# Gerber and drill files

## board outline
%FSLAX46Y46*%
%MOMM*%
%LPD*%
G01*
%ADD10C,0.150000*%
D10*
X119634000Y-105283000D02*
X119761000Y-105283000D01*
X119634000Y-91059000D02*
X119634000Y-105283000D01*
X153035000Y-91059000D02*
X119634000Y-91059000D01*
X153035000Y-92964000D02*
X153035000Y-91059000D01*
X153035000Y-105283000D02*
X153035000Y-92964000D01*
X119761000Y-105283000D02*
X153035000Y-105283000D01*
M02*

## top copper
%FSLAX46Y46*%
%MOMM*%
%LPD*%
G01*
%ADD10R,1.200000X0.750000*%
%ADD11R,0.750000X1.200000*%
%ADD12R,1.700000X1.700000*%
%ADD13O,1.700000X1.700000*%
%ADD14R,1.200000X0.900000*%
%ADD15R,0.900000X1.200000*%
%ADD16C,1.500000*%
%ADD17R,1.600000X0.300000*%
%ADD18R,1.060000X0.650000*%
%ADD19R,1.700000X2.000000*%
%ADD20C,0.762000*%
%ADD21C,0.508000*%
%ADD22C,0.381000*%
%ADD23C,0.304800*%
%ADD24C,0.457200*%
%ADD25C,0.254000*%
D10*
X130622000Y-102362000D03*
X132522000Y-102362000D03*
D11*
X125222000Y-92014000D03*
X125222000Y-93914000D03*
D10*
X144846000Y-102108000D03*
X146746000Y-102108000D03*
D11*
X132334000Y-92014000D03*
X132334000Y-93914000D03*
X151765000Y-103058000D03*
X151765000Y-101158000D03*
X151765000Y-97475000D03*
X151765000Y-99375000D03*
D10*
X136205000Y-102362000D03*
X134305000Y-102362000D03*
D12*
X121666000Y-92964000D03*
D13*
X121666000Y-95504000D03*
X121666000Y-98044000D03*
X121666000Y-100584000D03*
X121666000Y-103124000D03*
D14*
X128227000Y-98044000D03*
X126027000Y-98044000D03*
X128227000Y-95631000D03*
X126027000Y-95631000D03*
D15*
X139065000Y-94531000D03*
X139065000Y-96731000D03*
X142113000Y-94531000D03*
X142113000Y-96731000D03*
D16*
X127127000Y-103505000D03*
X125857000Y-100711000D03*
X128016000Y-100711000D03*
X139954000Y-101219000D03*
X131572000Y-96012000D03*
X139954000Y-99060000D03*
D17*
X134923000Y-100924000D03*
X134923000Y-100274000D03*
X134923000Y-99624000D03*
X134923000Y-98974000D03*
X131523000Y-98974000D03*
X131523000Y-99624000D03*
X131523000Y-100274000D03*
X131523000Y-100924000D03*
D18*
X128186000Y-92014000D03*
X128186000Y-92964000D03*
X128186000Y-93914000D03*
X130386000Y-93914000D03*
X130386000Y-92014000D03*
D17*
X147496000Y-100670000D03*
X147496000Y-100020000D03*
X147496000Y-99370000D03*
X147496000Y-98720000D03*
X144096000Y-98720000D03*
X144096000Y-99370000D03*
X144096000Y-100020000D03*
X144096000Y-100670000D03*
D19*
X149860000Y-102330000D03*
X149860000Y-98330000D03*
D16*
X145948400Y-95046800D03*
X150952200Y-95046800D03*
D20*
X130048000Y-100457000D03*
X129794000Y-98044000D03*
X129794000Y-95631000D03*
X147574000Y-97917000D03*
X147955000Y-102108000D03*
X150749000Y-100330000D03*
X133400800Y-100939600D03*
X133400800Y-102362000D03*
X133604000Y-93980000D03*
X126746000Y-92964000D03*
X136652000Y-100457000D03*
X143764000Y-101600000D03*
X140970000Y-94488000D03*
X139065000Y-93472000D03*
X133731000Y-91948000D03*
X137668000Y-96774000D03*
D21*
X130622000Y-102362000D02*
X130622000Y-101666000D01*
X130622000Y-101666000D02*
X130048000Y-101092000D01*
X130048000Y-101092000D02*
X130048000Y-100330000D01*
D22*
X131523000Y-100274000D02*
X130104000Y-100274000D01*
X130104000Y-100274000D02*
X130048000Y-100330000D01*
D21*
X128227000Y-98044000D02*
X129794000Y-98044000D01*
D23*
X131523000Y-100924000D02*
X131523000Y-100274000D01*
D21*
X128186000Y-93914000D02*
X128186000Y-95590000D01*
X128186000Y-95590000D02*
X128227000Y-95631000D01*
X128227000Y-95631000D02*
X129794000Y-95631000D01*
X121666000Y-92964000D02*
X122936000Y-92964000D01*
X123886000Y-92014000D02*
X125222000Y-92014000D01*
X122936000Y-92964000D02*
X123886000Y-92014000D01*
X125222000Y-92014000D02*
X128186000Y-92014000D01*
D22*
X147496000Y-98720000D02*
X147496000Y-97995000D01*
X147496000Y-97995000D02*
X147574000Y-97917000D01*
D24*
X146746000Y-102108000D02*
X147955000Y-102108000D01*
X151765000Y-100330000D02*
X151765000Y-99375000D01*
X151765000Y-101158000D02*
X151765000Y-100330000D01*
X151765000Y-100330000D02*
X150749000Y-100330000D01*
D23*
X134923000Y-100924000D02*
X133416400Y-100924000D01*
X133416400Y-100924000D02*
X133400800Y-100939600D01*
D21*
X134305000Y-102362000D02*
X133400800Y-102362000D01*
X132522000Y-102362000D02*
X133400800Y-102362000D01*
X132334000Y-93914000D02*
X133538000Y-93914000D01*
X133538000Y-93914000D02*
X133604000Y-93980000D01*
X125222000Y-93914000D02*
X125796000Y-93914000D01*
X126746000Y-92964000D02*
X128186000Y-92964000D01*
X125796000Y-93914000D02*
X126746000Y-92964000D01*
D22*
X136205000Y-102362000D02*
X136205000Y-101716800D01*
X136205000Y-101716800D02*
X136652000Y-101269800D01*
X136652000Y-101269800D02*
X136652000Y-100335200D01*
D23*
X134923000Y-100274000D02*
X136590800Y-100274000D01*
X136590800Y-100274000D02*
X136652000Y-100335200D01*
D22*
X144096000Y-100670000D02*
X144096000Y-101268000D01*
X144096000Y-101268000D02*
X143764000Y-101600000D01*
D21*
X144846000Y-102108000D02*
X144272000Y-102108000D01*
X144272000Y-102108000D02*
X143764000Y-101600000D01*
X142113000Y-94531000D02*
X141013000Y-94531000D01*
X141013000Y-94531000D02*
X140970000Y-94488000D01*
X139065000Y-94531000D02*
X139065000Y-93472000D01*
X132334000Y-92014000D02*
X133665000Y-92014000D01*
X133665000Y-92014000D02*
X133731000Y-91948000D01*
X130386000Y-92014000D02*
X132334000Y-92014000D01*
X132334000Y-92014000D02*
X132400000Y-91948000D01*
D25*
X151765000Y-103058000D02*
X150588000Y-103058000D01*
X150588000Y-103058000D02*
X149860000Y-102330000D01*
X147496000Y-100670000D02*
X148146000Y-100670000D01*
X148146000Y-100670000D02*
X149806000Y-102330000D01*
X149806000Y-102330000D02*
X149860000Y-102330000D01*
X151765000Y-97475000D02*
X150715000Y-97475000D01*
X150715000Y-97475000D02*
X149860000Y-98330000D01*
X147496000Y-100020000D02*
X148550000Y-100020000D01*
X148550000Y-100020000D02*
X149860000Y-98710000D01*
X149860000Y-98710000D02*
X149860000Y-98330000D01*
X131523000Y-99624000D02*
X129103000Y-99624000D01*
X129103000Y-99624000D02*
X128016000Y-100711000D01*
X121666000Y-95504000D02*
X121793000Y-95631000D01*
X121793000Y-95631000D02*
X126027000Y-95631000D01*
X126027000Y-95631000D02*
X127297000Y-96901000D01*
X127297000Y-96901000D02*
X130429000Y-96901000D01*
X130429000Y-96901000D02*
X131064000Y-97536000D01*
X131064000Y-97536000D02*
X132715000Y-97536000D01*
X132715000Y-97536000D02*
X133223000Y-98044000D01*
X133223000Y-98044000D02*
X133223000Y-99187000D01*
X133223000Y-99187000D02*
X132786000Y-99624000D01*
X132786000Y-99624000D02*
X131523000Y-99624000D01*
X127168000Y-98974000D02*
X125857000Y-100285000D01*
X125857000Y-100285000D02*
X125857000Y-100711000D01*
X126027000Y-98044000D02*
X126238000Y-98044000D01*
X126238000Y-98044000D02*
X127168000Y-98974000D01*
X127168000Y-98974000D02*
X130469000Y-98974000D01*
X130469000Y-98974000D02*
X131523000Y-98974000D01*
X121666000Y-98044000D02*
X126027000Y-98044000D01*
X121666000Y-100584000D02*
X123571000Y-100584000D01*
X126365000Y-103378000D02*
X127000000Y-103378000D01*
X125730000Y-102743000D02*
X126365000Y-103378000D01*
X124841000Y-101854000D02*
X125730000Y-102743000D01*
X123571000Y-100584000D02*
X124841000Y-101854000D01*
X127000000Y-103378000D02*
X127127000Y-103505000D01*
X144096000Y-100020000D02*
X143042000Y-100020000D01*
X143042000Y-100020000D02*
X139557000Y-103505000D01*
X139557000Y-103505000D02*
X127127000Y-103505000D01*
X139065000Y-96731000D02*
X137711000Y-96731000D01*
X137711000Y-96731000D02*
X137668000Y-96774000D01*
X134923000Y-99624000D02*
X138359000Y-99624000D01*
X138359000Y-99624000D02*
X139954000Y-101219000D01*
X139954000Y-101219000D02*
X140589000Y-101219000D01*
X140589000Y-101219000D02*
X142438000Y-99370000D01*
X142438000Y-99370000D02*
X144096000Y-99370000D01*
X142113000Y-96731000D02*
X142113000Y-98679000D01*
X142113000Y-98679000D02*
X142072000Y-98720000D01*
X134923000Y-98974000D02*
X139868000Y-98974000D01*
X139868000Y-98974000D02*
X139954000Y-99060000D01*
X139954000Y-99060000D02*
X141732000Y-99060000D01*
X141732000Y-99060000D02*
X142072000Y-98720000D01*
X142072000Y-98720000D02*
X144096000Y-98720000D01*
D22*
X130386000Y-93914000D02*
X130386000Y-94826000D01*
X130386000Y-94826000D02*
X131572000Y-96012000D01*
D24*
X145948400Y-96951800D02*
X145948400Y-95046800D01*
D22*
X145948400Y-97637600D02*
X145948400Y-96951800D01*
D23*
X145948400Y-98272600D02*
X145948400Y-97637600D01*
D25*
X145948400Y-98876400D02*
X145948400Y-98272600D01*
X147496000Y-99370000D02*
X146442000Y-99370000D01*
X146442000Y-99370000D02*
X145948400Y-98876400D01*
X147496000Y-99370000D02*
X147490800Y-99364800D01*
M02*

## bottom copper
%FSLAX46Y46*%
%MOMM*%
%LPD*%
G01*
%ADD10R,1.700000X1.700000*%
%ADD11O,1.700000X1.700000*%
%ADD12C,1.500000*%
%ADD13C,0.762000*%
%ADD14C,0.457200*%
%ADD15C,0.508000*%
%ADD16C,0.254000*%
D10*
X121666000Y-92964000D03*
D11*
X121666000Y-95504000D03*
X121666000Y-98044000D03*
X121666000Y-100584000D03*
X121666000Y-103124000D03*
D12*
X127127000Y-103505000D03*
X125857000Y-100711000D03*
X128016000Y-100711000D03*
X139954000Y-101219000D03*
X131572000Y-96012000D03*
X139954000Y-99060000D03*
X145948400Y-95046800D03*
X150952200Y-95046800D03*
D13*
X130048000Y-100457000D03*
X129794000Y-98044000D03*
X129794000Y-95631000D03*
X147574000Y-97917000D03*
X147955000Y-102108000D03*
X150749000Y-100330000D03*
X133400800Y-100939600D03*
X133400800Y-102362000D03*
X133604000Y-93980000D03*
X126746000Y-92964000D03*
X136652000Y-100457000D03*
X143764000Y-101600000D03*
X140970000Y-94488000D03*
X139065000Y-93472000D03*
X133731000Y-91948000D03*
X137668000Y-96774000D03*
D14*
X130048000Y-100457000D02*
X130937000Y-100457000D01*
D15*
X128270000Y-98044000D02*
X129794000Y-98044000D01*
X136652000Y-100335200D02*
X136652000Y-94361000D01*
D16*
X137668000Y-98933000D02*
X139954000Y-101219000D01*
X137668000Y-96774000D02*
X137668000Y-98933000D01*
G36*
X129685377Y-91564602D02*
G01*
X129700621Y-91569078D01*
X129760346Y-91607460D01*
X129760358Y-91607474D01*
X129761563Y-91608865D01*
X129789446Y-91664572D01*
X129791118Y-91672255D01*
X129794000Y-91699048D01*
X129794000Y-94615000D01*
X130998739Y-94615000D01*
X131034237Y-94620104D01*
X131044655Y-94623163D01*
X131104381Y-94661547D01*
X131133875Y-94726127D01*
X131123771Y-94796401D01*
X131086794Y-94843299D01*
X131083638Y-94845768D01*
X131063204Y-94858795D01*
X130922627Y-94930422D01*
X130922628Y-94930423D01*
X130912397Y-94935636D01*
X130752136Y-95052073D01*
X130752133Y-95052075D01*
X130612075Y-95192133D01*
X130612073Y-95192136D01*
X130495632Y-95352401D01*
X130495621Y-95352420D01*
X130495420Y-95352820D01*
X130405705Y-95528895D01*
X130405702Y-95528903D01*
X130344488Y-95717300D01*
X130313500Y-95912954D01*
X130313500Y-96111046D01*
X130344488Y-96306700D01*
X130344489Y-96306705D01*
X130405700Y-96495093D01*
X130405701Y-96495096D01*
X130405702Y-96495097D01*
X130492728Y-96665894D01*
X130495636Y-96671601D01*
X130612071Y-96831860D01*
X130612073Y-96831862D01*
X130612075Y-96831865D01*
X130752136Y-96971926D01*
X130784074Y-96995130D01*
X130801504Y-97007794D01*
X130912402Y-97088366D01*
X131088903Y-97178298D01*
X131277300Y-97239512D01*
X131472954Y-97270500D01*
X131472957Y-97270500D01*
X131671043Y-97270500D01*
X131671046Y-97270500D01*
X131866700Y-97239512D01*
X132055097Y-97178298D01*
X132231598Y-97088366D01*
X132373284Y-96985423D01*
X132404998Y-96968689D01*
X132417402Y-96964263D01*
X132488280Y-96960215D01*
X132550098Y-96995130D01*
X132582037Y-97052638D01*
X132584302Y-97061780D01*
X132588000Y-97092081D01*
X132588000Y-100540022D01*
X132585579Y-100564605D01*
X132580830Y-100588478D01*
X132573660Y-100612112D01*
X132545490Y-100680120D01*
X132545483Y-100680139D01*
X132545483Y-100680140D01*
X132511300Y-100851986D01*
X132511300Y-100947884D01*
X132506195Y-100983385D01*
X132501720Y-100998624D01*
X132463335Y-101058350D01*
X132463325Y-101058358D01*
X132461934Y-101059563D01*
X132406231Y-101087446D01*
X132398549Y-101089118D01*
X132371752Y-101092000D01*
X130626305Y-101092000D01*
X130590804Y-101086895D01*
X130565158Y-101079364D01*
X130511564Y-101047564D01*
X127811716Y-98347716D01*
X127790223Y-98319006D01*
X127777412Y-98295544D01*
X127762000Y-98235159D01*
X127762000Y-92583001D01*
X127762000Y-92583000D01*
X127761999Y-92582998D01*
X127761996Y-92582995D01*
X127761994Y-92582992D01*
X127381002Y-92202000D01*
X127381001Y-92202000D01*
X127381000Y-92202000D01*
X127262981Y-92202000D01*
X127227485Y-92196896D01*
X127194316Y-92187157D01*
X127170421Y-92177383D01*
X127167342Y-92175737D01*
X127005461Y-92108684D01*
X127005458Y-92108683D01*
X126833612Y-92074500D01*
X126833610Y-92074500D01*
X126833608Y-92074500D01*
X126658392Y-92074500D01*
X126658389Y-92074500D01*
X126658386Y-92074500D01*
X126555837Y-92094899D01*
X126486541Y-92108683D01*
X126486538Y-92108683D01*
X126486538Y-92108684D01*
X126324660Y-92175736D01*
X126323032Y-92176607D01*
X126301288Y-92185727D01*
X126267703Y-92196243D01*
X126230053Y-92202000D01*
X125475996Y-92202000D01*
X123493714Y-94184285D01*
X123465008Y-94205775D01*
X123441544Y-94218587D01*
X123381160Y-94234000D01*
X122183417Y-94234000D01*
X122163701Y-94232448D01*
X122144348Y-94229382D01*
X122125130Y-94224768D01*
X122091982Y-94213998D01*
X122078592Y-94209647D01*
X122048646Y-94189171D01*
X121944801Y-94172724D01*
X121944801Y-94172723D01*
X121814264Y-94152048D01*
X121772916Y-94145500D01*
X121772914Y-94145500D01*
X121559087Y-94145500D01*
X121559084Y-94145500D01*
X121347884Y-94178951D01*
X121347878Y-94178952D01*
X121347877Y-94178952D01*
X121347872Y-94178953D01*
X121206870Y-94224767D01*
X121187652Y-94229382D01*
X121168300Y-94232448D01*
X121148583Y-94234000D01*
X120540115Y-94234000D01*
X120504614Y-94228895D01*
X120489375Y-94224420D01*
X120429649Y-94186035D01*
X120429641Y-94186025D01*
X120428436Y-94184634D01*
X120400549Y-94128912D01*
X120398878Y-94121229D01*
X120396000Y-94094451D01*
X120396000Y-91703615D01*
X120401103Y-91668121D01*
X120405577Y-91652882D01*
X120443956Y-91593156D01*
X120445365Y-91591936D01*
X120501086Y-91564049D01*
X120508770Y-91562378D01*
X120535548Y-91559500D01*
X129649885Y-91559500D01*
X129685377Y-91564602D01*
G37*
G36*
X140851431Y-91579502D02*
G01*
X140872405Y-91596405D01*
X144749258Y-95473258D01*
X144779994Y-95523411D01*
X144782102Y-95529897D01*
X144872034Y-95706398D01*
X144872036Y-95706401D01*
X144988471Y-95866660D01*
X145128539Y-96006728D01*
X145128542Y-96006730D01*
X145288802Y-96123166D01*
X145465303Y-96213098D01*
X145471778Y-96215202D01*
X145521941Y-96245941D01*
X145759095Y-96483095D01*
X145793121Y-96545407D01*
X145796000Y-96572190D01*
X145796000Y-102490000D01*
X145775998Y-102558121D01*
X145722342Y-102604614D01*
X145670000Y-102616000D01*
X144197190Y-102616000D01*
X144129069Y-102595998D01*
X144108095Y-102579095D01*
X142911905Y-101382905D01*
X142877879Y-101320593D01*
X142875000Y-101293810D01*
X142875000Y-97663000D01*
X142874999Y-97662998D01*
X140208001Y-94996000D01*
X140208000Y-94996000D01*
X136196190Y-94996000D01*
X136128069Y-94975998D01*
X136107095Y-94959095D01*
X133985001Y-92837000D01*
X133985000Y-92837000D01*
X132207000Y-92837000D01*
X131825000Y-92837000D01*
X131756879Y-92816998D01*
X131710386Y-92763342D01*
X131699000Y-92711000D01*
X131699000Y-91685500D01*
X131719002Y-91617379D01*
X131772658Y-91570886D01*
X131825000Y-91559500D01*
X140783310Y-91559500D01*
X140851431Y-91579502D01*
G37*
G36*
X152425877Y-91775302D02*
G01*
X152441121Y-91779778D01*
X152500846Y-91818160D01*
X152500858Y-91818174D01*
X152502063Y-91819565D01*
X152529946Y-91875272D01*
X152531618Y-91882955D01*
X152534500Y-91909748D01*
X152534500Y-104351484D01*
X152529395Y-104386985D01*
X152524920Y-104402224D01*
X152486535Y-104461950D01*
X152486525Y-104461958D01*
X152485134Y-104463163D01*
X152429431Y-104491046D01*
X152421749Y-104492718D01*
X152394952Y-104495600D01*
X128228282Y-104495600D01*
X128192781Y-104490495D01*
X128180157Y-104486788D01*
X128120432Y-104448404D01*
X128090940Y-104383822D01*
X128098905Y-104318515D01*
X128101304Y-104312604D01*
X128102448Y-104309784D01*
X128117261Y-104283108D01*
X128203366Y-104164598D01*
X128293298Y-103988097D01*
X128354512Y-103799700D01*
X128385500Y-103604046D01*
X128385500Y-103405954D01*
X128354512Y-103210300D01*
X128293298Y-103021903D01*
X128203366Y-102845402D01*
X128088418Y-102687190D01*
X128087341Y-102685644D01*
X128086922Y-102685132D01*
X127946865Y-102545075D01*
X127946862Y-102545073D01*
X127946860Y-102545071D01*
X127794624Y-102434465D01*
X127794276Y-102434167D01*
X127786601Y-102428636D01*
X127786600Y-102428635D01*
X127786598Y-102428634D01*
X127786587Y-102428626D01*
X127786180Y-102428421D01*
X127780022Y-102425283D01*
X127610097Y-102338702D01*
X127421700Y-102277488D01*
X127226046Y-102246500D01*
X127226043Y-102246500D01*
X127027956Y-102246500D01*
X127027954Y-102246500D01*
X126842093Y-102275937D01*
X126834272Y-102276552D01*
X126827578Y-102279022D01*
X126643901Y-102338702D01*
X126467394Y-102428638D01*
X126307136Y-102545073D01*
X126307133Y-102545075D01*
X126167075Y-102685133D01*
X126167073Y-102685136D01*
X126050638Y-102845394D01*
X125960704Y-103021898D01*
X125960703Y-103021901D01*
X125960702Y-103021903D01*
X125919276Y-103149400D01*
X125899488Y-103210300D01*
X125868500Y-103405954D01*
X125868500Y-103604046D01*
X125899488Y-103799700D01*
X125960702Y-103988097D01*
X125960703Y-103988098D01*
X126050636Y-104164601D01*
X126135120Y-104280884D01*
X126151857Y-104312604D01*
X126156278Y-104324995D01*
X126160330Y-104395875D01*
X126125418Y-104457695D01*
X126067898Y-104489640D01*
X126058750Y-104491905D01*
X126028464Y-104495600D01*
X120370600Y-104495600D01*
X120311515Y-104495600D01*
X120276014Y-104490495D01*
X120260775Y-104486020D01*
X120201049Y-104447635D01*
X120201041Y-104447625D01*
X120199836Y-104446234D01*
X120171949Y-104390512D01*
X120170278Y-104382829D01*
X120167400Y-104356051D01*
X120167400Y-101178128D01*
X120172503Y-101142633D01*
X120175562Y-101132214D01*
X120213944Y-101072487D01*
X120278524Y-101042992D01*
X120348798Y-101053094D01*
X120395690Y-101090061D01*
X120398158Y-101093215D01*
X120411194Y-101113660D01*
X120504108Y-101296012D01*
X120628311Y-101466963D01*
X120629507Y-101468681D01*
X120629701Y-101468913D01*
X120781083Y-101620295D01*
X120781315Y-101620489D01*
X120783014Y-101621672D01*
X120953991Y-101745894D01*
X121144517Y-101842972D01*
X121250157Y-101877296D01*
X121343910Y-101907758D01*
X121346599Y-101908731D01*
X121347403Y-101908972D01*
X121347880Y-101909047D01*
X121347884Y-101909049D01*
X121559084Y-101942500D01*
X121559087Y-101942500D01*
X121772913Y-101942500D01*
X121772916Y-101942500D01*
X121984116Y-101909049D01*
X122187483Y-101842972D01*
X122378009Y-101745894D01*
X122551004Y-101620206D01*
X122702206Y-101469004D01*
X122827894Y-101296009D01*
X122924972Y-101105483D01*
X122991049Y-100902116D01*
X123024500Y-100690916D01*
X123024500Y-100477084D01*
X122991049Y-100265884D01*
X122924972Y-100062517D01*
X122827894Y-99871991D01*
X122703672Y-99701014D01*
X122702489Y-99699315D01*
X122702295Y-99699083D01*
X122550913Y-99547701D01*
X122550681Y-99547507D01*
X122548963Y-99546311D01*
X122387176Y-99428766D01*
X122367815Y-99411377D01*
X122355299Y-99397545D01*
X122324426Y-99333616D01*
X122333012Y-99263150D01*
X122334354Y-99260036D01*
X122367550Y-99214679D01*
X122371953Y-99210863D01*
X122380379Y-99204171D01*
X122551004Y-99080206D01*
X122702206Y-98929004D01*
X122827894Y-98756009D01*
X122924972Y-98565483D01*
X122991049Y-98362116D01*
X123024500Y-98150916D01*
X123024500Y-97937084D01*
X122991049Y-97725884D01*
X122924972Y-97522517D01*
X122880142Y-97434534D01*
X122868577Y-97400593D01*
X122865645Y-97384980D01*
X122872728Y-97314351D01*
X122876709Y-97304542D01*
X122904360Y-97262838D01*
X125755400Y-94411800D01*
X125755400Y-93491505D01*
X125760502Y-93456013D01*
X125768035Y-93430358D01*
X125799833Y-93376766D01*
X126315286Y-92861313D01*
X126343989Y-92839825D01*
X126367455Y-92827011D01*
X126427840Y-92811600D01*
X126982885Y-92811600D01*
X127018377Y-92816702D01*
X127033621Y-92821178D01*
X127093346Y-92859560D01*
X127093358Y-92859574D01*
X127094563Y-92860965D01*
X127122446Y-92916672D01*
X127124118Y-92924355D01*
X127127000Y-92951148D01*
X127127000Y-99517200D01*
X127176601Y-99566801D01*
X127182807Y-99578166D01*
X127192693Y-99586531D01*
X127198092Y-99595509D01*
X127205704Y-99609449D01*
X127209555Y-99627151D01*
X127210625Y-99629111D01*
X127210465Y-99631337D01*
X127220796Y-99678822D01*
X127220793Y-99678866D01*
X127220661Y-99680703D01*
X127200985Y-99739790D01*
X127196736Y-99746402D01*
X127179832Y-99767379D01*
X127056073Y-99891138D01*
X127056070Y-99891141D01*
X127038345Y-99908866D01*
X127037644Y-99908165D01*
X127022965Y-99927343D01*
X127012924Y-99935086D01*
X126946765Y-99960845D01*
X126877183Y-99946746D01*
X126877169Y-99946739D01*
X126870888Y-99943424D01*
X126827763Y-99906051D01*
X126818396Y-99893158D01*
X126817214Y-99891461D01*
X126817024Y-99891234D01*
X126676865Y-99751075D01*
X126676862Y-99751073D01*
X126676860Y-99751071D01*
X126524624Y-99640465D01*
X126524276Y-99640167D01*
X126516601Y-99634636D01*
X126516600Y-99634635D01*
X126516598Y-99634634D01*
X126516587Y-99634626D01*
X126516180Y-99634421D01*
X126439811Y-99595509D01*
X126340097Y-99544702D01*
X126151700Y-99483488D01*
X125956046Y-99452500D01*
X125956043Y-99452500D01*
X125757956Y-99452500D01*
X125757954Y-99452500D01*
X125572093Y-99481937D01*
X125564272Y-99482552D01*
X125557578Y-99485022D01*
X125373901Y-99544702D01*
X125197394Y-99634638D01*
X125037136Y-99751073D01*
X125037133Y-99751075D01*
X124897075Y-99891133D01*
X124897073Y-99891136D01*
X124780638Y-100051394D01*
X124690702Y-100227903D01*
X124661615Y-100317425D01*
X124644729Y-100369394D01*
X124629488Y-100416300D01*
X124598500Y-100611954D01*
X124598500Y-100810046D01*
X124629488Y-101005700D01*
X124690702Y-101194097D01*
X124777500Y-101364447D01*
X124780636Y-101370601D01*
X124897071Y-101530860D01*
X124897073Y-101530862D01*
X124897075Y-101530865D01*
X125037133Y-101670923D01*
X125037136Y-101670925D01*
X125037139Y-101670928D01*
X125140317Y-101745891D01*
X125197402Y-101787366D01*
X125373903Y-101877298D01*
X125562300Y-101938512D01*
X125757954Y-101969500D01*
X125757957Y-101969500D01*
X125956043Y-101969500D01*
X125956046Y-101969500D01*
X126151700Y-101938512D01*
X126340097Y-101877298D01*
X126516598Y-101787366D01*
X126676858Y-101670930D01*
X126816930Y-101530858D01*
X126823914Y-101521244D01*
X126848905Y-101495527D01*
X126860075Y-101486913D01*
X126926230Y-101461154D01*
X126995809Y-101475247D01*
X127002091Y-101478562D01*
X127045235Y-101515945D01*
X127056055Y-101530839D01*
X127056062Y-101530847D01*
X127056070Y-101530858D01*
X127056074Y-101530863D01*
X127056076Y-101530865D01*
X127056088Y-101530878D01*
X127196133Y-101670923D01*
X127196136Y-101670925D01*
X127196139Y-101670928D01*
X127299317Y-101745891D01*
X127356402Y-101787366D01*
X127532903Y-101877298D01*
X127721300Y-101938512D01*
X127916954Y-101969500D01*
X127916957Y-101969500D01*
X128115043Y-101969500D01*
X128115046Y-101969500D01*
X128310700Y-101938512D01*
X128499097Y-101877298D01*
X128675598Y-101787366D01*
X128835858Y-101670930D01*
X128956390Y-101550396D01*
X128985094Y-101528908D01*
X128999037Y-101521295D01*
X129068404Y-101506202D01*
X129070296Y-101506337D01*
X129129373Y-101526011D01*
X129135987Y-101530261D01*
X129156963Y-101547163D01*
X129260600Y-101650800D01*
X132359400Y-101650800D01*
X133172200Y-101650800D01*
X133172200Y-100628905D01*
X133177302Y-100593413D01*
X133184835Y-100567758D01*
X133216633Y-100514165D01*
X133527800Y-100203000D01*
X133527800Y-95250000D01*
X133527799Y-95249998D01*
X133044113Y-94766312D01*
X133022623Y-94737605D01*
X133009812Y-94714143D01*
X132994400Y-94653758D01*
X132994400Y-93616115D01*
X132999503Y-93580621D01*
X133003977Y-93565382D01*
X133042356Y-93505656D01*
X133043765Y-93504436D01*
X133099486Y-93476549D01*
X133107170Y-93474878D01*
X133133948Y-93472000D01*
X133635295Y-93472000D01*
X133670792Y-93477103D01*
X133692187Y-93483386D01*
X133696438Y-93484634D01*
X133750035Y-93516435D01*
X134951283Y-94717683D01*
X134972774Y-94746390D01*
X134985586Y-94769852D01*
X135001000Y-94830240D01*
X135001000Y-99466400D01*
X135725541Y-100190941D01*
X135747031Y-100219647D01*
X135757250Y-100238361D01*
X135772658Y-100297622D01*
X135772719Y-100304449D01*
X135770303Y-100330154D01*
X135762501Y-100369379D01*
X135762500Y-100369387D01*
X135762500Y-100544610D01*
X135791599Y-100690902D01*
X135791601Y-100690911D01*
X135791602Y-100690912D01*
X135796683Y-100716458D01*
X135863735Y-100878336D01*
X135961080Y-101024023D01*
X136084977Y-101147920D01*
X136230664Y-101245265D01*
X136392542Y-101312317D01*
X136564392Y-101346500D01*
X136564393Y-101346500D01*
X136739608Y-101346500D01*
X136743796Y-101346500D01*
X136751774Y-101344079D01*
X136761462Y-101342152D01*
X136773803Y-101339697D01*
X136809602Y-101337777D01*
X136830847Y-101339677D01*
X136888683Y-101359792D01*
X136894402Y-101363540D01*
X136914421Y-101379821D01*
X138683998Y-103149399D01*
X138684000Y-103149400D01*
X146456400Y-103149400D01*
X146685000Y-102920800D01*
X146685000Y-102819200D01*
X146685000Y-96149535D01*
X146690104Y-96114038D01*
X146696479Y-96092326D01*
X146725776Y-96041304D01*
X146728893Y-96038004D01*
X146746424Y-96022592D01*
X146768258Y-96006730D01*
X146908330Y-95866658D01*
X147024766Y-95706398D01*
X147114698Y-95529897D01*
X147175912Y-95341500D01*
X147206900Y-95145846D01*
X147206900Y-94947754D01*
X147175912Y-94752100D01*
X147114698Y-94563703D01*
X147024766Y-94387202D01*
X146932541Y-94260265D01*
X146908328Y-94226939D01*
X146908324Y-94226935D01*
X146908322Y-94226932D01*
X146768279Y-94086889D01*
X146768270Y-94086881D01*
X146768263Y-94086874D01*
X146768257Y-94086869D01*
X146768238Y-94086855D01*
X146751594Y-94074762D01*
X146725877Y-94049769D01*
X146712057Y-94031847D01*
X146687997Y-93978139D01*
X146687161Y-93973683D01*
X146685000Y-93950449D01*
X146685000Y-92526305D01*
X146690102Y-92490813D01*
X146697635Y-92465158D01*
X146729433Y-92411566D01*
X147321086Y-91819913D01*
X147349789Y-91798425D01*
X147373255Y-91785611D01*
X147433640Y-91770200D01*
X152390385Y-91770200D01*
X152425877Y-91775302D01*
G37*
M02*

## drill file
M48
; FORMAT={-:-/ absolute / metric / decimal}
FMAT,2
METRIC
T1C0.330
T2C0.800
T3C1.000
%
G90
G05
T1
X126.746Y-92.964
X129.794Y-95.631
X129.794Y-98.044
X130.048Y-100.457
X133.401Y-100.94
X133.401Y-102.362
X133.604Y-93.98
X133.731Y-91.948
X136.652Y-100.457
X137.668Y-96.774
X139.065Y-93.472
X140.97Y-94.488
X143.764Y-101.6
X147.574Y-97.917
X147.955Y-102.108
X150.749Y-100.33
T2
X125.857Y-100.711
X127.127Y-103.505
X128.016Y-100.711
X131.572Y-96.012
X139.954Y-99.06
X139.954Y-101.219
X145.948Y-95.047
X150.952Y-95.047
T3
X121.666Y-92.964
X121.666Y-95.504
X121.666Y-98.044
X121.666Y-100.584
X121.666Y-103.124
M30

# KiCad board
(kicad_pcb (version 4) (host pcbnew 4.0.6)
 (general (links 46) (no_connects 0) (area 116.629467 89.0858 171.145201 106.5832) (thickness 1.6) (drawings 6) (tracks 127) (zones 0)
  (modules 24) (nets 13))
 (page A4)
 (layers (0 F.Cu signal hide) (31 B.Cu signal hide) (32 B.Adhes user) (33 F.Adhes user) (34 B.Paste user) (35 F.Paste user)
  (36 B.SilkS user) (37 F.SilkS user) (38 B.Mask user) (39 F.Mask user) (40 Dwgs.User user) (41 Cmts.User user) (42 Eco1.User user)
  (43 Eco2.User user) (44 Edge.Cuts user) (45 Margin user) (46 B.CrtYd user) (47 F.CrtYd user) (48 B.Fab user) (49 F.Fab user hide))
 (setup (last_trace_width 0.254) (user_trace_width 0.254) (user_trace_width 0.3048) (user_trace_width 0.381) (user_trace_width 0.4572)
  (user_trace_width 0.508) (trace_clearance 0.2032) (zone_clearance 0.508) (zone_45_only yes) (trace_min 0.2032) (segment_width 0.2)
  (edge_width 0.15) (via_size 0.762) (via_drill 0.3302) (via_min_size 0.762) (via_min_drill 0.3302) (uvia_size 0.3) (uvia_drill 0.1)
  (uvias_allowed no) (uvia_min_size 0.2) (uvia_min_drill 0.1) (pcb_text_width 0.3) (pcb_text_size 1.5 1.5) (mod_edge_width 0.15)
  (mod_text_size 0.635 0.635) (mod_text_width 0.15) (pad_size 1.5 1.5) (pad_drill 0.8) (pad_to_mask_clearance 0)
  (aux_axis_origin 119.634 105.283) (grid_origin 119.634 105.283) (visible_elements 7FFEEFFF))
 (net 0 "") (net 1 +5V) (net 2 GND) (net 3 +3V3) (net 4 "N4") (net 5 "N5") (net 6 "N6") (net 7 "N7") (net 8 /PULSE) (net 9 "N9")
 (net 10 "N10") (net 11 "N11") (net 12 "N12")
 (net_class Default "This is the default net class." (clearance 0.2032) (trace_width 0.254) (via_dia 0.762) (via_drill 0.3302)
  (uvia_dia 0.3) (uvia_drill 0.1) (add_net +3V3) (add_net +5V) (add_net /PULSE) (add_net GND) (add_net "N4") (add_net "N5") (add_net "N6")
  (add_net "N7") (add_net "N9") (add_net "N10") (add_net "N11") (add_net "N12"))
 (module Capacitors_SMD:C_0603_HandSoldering (layer F.Cu) (at 131.572 102.362)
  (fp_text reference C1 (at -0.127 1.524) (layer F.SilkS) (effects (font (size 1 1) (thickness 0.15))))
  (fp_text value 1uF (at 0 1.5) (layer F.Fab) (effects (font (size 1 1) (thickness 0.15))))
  (pad 1 smd rect (at -0.95 0) (size 1.2 0.75) (layers F.Cu F.Paste F.Mask) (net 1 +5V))
  (pad 2 smd rect (at 0.95 0) (size 1.2 0.75) (layers F.Cu F.Paste F.Mask) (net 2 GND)))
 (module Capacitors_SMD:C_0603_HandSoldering (layer F.Cu) (at 125.222 92.964 270)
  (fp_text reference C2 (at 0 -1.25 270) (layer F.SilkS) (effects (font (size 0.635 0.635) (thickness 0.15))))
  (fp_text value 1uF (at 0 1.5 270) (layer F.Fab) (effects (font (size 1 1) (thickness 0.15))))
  (pad 1 smd rect (at -0.95 0 270) (size 1.2 0.75) (layers F.Cu F.Paste F.Mask) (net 1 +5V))
  (pad 2 smd rect (at 0.95 0 270) (size 1.2 0.75) (layers F.Cu F.Paste F.Mask) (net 2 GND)))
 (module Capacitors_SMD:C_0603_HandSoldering (layer F.Cu) (at 145.796 102.108)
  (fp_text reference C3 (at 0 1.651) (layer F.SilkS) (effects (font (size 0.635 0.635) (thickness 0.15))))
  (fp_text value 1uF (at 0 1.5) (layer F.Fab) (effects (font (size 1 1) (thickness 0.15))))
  (pad 1 smd rect (at -0.95 0) (size 1.2 0.75) (layers F.Cu F.Paste F.Mask) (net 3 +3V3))
  (pad 2 smd rect (at 0.95 0) (size 1.2 0.75) (layers F.Cu F.Paste F.Mask) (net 2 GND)))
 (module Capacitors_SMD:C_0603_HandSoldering (layer F.Cu) (at 132.334 92.964 270)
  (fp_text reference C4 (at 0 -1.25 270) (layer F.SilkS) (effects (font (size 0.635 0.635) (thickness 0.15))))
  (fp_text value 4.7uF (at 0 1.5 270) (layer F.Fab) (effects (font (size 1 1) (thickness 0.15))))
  (pad 1 smd rect (at -0.95 0 270) (size 1.2 0.75) (layers F.Cu F.Paste F.Mask) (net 3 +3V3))
  (pad 2 smd rect (at 0.95 0 270) (size 1.2 0.75) (layers F.Cu F.Paste F.Mask) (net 2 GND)))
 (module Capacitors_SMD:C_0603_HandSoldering (layer F.Cu) (at 151.765 102.108 90)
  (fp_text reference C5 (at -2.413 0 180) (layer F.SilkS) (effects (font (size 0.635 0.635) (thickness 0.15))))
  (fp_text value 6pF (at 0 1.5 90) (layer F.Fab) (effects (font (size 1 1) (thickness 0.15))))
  (pad 1 smd rect (at -0.95 0 90) (size 1.2 0.75) (layers F.Cu F.Paste F.Mask) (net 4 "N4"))
  (pad 2 smd rect (at 0.95 0 90) (size 1.2 0.75) (layers F.Cu F.Paste F.Mask) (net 2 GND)))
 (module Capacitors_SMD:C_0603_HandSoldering (layer F.Cu) (at 151.765 98.425 270)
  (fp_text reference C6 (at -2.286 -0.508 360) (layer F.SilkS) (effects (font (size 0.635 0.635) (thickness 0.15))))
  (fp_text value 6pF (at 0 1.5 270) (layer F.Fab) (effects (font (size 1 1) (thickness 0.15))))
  (pad 1 smd rect (at -0.95 0 270) (size 1.2 0.75) (layers F.Cu F.Paste F.Mask) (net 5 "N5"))
  (pad 2 smd rect (at 0.95 0 270) (size 1.2 0.75) (layers F.Cu F.Paste F.Mask) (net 2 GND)))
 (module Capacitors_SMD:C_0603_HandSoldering (layer F.Cu) (at 135.255 102.362 180)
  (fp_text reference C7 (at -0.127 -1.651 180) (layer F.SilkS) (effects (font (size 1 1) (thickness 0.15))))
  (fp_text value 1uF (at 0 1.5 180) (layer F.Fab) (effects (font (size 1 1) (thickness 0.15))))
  (pad 1 smd rect (at -0.95 0 180) (size 1.2 0.75) (layers F.Cu F.Paste F.Mask) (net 3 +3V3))
  (pad 2 smd rect (at 0.95 0 180) (size 1.2 0.75) (layers F.Cu F.Paste F.Mask) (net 2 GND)))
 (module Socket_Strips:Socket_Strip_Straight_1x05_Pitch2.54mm (layer F.Cu) (at 121.666 92.964)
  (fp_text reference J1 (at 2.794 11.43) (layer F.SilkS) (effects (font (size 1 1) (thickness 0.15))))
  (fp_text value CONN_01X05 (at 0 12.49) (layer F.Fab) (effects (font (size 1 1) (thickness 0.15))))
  (pad 1 thru_hole rect (at 0 0) (size 1.7 1.7) (drill 1) (layers *.Cu *.Mask) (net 1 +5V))
  (pad 2 thru_hole oval (at 0 2.54) (size 1.7 1.7) (drill 1) (layers *.Cu *.Mask) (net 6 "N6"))
  (pad 3 thru_hole oval (at 0 5.08) (size 1.7 1.7) (drill 1) (layers *.Cu *.Mask) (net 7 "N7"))
  (pad 4 thru_hole oval (at 0 7.62) (size 1.7 1.7) (drill 1) (layers *.Cu *.Mask) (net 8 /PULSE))
  (pad 5 thru_hole oval (at 0 10.16) (size 1.7 1.7) (drill 1) (layers *.Cu *.Mask) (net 2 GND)))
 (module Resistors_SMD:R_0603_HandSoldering (layer F.Cu) (at 127.127 98.044 180)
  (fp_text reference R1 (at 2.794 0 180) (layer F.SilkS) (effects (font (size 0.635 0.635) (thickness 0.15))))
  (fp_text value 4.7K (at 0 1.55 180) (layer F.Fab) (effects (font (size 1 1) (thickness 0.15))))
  (pad 1 smd rect (at -1.1 0 180) (size 1.2 0.9) (layers F.Cu F.Paste F.Mask) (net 1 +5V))
  (pad 2 smd rect (at 1.1 0 180) (size 1.2 0.9) (layers F.Cu F.Paste F.Mask) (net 7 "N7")))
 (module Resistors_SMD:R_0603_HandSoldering (layer F.Cu) (at 127.127 95.631 180)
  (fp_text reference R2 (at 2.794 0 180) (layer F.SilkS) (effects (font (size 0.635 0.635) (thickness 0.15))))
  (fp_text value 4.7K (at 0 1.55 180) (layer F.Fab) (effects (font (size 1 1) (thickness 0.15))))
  (pad 1 smd rect (at -1.1 0 180) (size 1.2 0.9) (layers F.Cu F.Paste F.Mask) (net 1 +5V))
  (pad 2 smd rect (at 1.1 0 180) (size 1.2 0.9) (layers F.Cu F.Paste F.Mask) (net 6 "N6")))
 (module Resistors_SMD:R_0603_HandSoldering (layer F.Cu) (at 139.065 95.631 270)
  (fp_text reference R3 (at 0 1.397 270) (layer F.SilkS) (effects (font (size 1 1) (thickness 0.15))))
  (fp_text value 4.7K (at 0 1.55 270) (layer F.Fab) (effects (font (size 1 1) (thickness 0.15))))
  (pad 1 smd rect (at -1.1 0 270) (size 1.2 0.9) (layers F.Cu F.Paste F.Mask) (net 3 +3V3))
  (pad 2 smd rect (at 1.1 0 270) (size 1.2 0.9) (layers F.Cu F.Paste F.Mask) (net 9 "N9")))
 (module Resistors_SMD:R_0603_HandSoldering (layer F.Cu) (at 142.113 95.631 270)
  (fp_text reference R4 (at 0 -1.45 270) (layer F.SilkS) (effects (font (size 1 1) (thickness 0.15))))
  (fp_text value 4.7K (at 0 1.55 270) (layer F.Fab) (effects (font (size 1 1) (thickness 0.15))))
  (pad 1 smd rect (at -1.1 0 270) (size 1.2 0.9) (layers F.Cu F.Paste F.Mask) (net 3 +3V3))
  (pad 2 smd rect (at 1.1 0 270) (size 1.2 0.9) (layers F.Cu F.Paste F.Mask) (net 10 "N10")))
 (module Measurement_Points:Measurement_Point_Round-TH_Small (layer F.Cu) (at 127.127 103.505)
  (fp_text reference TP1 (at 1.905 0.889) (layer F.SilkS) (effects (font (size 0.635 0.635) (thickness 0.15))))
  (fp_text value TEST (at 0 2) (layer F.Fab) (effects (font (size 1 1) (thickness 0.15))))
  (pad 1 thru_hole circle (at 0 0) (size 1.5 1.5) (drill 0.8) (layers *.Cu *.Mask) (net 8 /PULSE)))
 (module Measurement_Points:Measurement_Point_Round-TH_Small (layer F.Cu) (at 125.857 100.711)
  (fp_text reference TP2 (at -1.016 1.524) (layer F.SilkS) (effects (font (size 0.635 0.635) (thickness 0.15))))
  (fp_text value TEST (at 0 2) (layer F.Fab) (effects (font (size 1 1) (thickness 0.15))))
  (pad 1 thru_hole circle (at 0 0) (size 1.5 1.5) (drill 0.8) (layers *.Cu *.Mask) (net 7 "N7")))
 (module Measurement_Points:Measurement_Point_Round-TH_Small (layer F.Cu) (at 128.016 100.711)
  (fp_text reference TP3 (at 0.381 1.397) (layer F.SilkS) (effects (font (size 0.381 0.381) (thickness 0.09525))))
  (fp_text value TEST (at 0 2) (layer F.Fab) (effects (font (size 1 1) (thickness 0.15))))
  (pad 1 thru_hole circle (at 0 0) (size 1.5 1.5) (drill 0.8) (layers *.Cu *.Mask) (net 6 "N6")))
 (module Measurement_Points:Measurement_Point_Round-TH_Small (layer F.Cu) (at 139.954 101.219)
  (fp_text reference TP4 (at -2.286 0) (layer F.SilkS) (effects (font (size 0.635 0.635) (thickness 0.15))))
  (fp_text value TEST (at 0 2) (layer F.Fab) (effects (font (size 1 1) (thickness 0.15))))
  (pad 1 thru_hole circle (at 0 0) (size 1.5 1.5) (drill 0.8) (layers *.Cu *.Mask) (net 9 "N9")))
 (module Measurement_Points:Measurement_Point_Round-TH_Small (layer F.Cu) (at 131.572 96.012)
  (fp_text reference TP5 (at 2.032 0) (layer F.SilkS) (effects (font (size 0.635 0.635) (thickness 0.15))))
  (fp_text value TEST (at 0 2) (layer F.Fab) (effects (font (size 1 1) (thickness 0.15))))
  (pad 1 thru_hole circle (at 0 0) (size 1.5 1.5) (drill 0.8) (layers *.Cu *.Mask) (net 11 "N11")))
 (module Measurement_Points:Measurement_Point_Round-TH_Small (layer F.Cu) (at 139.954 99.06)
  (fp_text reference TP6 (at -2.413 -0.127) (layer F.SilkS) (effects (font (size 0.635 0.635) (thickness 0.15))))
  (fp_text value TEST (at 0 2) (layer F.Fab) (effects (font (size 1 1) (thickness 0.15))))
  (pad 1 thru_hole circle (at 0 0) (size 1.5 1.5) (drill 0.8) (layers *.Cu *.Mask) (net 10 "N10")))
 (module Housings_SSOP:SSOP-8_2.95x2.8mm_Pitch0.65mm (layer F.Cu) (at 133.223 99.949 180)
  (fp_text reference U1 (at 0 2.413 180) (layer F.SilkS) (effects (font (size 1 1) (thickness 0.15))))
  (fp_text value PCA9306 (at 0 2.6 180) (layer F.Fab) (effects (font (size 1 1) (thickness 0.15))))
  (pad 1 smd rect (at -1.7 -0.975 90) (size 0.3 1.6) (layers F.Cu F.Paste F.Mask) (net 2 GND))
  (pad 2 smd rect (at -1.7 -0.325 90) (size 0.3 1.6) (layers F.Cu F.Paste F.Mask) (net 3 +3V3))
  (pad 3 smd rect (at -1.7 0.325 90) (size 0.3 1.6) (layers F.Cu F.Paste F.Mask) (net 9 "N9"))
  (pad 4 smd rect (at -1.7 0.975 90) (size 0.3 1.6) (layers F.Cu F.Paste F.Mask) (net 10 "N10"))
  (pad 5 smd rect (at 1.7 0.975 90) (size 0.3 1.6) (layers F.Cu F.Paste F.Mask) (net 7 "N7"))
  (pad 6 smd rect (at 1.7 0.325 90) (size 0.3 1.6) (layers F.Cu F.Paste F.Mask) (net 6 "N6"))
  (pad 7 smd rect (at 1.7 -0.325 90) (size 0.3 1.6) (layers F.Cu F.Paste F.Mask) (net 1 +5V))
  (pad 8 smd rect (at 1.7 -0.975 90) (size 0.3 1.6) (layers F.Cu F.Paste F.Mask) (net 1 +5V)))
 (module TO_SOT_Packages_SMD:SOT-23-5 (layer F.Cu) (at 129.286 92.964)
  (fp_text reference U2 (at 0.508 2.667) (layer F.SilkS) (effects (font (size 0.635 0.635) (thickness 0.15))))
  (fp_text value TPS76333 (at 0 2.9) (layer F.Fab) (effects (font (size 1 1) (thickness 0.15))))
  (pad 1 smd rect (at -1.1 -0.95) (size 1.06 0.65) (layers F.Cu F.Paste F.Mask) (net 1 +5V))
  (pad 2 smd rect (at -1.1 0) (size 1.06 0.65) (layers F.Cu F.Paste F.Mask) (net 2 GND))
  (pad 3 smd rect (at -1.1 0.95) (size 1.06 0.65) (layers F.Cu F.Paste F.Mask) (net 1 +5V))
  (pad 4 smd rect (at 1.1 0.95) (size 1.06 0.65) (layers F.Cu F.Paste F.Mask) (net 11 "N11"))
  (pad 5 smd rect (at 1.1 -0.95) (size 1.06 0.65) (layers F.Cu F.Paste F.Mask) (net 3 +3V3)))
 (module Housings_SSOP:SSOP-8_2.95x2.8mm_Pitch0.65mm (layer F.Cu) (at 145.796 99.695 180)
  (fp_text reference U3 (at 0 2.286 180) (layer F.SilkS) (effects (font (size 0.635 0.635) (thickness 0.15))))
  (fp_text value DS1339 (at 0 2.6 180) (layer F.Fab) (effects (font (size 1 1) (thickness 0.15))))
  (pad 1 smd rect (at -1.7 -0.975 90) (size 0.3 1.6) (layers F.Cu F.Paste F.Mask) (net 4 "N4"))
  (pad 2 smd rect (at -1.7 -0.325 90) (size 0.3 1.6) (layers F.Cu F.Paste F.Mask) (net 5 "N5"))
  (pad 3 smd rect (at -1.7 0.325 90) (size 0.3 1.6) (layers F.Cu F.Paste F.Mask) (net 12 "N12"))
  (pad 4 smd rect (at -1.7 0.975 90) (size 0.3 1.6) (layers F.Cu F.Paste F.Mask) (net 2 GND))
  (pad 5 smd rect (at 1.7 0.975 90) (size 0.3 1.6) (layers F.Cu F.Paste F.Mask) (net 10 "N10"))
  (pad 6 smd rect (at 1.7 0.325 90) (size 0.3 1.6) (layers F.Cu F.Paste F.Mask) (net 9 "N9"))
  (pad 7 smd rect (at 1.7 -0.325 90) (size 0.3 1.6) (layers F.Cu F.Paste F.Mask) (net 8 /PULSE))
  (pad 8 smd rect (at 1.7 -0.975 90) (size 0.3 1.6) (layers F.Cu F.Paste F.Mask) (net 3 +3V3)))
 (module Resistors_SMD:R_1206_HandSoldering (layer F.Cu) (at 149.86 100.33 90)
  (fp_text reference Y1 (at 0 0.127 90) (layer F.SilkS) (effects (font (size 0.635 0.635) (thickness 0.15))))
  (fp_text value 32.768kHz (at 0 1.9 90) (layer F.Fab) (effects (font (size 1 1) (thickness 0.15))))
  (pad 1 smd rect (at -2 0 90) (size 2 1.7) (layers F.Cu F.Paste F.Mask) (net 4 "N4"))
  (pad 2 smd rect (at 2 0 90) (size 2 1.7) (layers F.Cu F.Paste F.Mask) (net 5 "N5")))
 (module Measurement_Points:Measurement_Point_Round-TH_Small (layer F.Cu) (at 145.9484 95.0468)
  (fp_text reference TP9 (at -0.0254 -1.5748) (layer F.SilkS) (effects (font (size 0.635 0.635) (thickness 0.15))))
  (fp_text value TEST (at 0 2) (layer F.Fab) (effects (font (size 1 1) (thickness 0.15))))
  (pad 1 thru_hole circle (at 0 0) (size 1.5 1.5) (drill 0.8) (layers *.Cu *.Mask) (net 12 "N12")))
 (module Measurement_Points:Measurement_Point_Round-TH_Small (layer F.Cu) (at 150.9522 95.0468)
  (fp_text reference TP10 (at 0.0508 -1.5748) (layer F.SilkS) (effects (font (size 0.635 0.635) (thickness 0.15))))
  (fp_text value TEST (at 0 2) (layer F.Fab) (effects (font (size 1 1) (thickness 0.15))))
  (pad 1 thru_hole circle (at 0 0) (size 1.5 1.5) (drill 0.8) (layers *.Cu *.Mask) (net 2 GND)))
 (gr_line (start 119.634 105.283) (end 119.761 105.283) (angle 90) (layer Edge.Cuts) (width 0.15))
 (gr_line (start 119.634 91.059) (end 119.634 105.283) (angle 90) (layer Edge.Cuts) (width 0.15))
 (gr_line (start 153.035 91.059) (end 119.634 91.059) (angle 90) (layer Edge.Cuts) (width 0.15))
 (gr_line (start 153.035 92.964) (end 153.035 91.059) (angle 90) (layer Edge.Cuts) (width 0.15))
 (gr_line (start 153.035 105.283) (end 153.035 92.964) (angle 90) (layer Edge.Cuts) (width 0.15))
 (gr_line (start 119.761 105.283) (end 153.035 105.283) (angle 90) (layer Edge.Cuts) (width 0.15))
 (segment (start 130.048 100.457) (end 130.937 100.457) (width 0.4572) (layer B.Cu) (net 1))
 (segment (start 130.622 102.362) (end 130.622 101.666) (width 0.508) (layer F.Cu) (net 1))
 (segment (start 130.622 101.666) (end 130.048 101.092) (width 0.508) (layer F.Cu) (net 1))
 (segment (start 130.048 101.092) (end 130.048 100.33) (width 0.508) (layer F.Cu) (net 1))
 (segment (start 131.523 100.274) (end 130.104 100.274) (width 0.381) (layer F.Cu) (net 1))
 (segment (start 130.104 100.274) (end 130.048 100.33) (width 0.381) (layer F.Cu) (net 1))
 (segment (start 128.227 98.044) (end 129.794 98.044) (width 0.508) (layer F.Cu) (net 1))
 (segment (start 131.523 100.924) (end 131.523 100.274) (width 0.3048) (layer F.Cu) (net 1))
 (via (at 130.048 100.457) (size 0.762) (drill 0.3302) (layers F.Cu B.Cu) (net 1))
 (segment (start 128.27 98.044) (end 129.794 98.044) (width 0.508) (layer B.Cu) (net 1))
 (via (at 129.794 98.044) (size 0.762) (drill 0.3302) (layers F.Cu B.Cu) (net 1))
 (segment (start 128.186 93.914) (end 128.186 95.59) (width 0.508) (layer F.Cu) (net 1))
 (segment (start 128.186 95.59) (end 128.227 95.631) (width 0.508) (layer F.Cu) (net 1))
 (segment (start 128.227 95.631) (end 129.794 95.631) (width 0.508) (layer F.Cu) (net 1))
 (via (at 129.794 95.631) (size 0.762) (drill 0.3302) (layers F.Cu B.Cu) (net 1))
 (segment (start 121.666 92.964) (end 122.936 92.964) (width 0.508) (layer F.Cu) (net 1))
 (segment (start 123.886 92.014) (end 125.222 92.014) (width 0.508) (layer F.Cu) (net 1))
 (segment (start 122.936 92.964) (end 123.886 92.014) (width 0.508) (layer F.Cu) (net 1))
 (segment (start 125.222 92.014) (end 128.186 92.014) (width 0.508) (layer F.Cu) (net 1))
 (segment (start 147.496 98.72) (end 147.496 97.995) (width 0.381) (layer F.Cu) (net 2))
 (segment (start 147.496 97.995) (end 147.574 97.917) (width 0.381) (layer F.Cu) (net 2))
 (via (at 147.574 97.917) (size 0.762) (drill 0.3302) (layers F.Cu B.Cu) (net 2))
 (segment (start 146.746 102.108) (end 147.955 102.108) (width 0.4572) (layer F.Cu) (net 2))
 (via (at 147.955 102.108) (size 0.762) (drill 0.3302) (layers F.Cu B.Cu) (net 2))
 (segment (start 151.765 100.33) (end 151.765 99.375) (width 0.4572) (layer F.Cu) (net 2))
 (segment (start 151.765 101.158) (end 151.765 100.33) (width 0.4572) (layer F.Cu) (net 2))
 (segment (start 151.765 100.33) (end 150.749 100.33) (width 0.4572) (layer F.Cu) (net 2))
 (via (at 150.749 100.33) (size 0.762) (drill 0.3302) (layers F.Cu B.Cu) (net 2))
 (segment (start 134.923 100.924) (end 133.4164 100.924) (width 0.3048) (layer F.Cu) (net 2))
 (segment (start 133.4164 100.924) (end 133.4008 100.9396) (width 0.3048) (layer F.Cu) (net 2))
 (via (at 133.4008 100.9396) (size 0.762) (drill 0.3302) (layers F.Cu B.Cu) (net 2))
 (segment (start 134.305 102.362) (end 133.4008 102.362) (width 0.508) (layer F.Cu) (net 2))
 (segment (start 132.522 102.362) (end 133.4008 102.362) (width 0.508) (layer F.Cu) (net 2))
 (via (at 133.4008 102.362) (size 0.762) (drill 0.3302) (layers F.Cu B.Cu) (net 2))
 (segment (start 132.334 93.914) (end 133.538 93.914) (width 0.508) (layer F.Cu) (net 2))
 (via (at 133.604 93.98) (size 0.762) (drill 0.3302) (layers F.Cu B.Cu) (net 2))
 (segment (start 133.538 93.914) (end 133.604 93.98) (width 0.508) (layer F.Cu) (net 2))
 (segment (start 125.222 93.914) (end 125.796 93.914) (width 0.508) (layer F.Cu) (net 2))
 (via (at 126.746 92.964) (size 0.762) (drill 0.3302) (layers F.Cu B.Cu) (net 2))
 (segment (start 126.746 92.964) (end 128.186 92.964) (width 0.508) (layer F.Cu) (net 2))
 (segment (start 125.796 93.914) (end 126.746 92.964) (width 0.508) (layer F.Cu) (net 2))
 (segment (start 136.205 102.362) (end 136.205 101.7168) (width 0.381) (layer F.Cu) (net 3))
 (segment (start 136.205 101.7168) (end 136.652 101.2698) (width 0.381) (layer F.Cu) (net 3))
 (segment (start 136.652 101.2698) (end 136.652 100.3352) (width 0.381) (layer F.Cu) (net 3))
 (segment (start 136.652 100.3352) (end 136.652 94.361) (width 0.508) (layer B.Cu) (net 3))
 (segment (start 134.923 100.274) (end 136.5908 100.274) (width 0.3048) (layer F.Cu) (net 3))
 (segment (start 136.5908 100.274) (end 136.652 100.3352) (width 0.3048) (layer F.Cu) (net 3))
 (via (at 136.652 100.457) (size 0.762) (drill 0.3302) (layers F.Cu B.Cu) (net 3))
 (segment (start 144.096 100.67) (end 144.096 101.268) (width 0.381) (layer F.Cu) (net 3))
 (segment (start 144.096 101.268) (end 143.764 101.6) (width 0.381) (layer F.Cu) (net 3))
 (segment (start 144.846 102.108) (end 144.272 102.108) (width 0.508) (layer F.Cu) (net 3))
 (segment (start 144.272 102.108) (end 143.764 101.6) (width 0.508) (layer F.Cu) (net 3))
 (via (at 143.764 101.6) (size 0.762) (drill 0.3302) (layers F.Cu B.Cu) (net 3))
 (segment (start 142.113 94.531) (end 141.013 94.531) (width 0.508) (layer F.Cu) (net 3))
 (segment (start 141.013 94.531) (end 140.97 94.488) (width 0.508) (layer F.Cu) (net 3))
 (via (at 140.97 94.488) (size 0.762) (drill 0.3302) (layers F.Cu B.Cu) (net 3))
 (segment (start 139.065 94.531) (end 139.065 93.472) (width 0.508) (layer F.Cu) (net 3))
 (via (at 139.065 93.472) (size 0.762) (drill 0.3302) (layers F.Cu B.Cu) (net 3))
 (segment (start 132.334 92.014) (end 133.665 92.014) (width 0.508) (layer F.Cu) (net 3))
 (segment (start 133.665 92.014) (end 133.731 91.948) (width 0.508) (layer F.Cu) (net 3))
 (via (at 133.731 91.948) (size 0.762) (drill 0.3302) (layers F.Cu B.Cu) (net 3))
 (segment (start 130.386 92.014) (end 132.334 92.014) (width 0.508) (layer F.Cu) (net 3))
 (segment (start 132.334 92.014) (end 132.4 91.948) (width 0.508) (layer F.Cu) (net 3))
 (segment (start 151.765 103.058) (end 150.588 103.058) (width 0.254) (layer F.Cu) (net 4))
 (segment (start 150.588 103.058) (end 149.86 102.33) (width 0.254) (layer F.Cu) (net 4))
 (segment (start 147.496 100.67) (end 148.146 100.67) (width 0.254) (layer F.Cu) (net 4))
 (segment (start 148.146 100.67) (end 149.806 102.33) (width 0.254) (layer F.Cu) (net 4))
 (segment (start 149.806 102.33) (end 149.86 102.33) (width 0.254) (layer F.Cu) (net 4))
 (segment (start 151.765 97.475) (end 150.715 97.475) (width 0.254) (layer F.Cu) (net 5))
 (segment (start 150.715 97.475) (end 149.86 98.33) (width 0.254) (layer F.Cu) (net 5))
 (segment (start 147.496 100.02) (end 148.55 100.02) (width 0.254) (layer F.Cu) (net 5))
 (segment (start 148.55 100.02) (end 149.86 98.71) (width 0.254) (layer F.Cu) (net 5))
 (segment (start 149.86 98.71) (end 149.86 98.33) (width 0.254) (layer F.Cu) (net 5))
 (segment (start 131.523 99.624) (end 129.103 99.624) (width 0.254) (layer F.Cu) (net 6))
 (segment (start 129.103 99.624) (end 128.016 100.711) (width 0.254) (layer F.Cu) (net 6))
 (segment (start 121.666 95.504) (end 121.793 95.631) (width 0.254) (layer F.Cu) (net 6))
 (segment (start 121.793 95.631) (end 126.027 95.631) (width 0.254) (layer F.Cu) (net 6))
 (segment (start 126.027 95.631) (end 127.297 96.901) (width 0.254) (layer F.Cu) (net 6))
 (segment (start 127.297 96.901) (end 130.429 96.901) (width 0.254) (layer F.Cu) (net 6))
 (segment (start 130.429 96.901) (end 131.064 97.536) (width 0.254) (layer F.Cu) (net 6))
 (segment (start 131.064 97.536) (end 132.715 97.536) (width 0.254) (layer F.Cu) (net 6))
 (segment (start 132.715 97.536) (end 133.223 98.044) (width 0.254) (layer F.Cu) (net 6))
 (segment (start 133.223 98.044) (end 133.223 99.187) (width 0.254) (layer F.Cu) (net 6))
 (segment (start 133.223 99.187) (end 132.786 99.624) (width 0.254) (layer F.Cu) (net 6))
 (segment (start 132.786 99.624) (end 131.523 99.624) (width 0.254) (layer F.Cu) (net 6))
 (segment (start 127.168 98.974) (end 125.857 100.285) (width 0.254) (layer F.Cu) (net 7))
 (segment (start 125.857 100.285) (end 125.857 100.711) (width 0.254) (layer F.Cu) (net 7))
 (segment (start 126.027 98.044) (end 126.238 98.044) (width 0.254) (layer F.Cu) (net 7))
 (segment (start 126.238 98.044) (end 127.168 98.974) (width 0.254) (layer F.Cu) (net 7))
 (segment (start 127.168 98.974) (end 130.469 98.974) (width 0.254) (layer F.Cu) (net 7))
 (segment (start 130.469 98.974) (end 131.523 98.974) (width 0.254) (layer F.Cu) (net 7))
 (segment (start 121.666 98.044) (end 126.027 98.044) (width 0.254) (layer F.Cu) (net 7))
 (segment (start 121.666 100.584) (end 123.571 100.584) (width 0.254) (layer F.Cu) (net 8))
 (segment (start 126.365 103.378) (end 127 103.378) (width 0.254) (layer F.Cu) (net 8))
 (segment (start 125.73 102.743) (end 126.365 103.378) (width 0.254) (layer F.Cu) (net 8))
 (segment (start 124.841 101.854) (end 125.73 102.743) (width 0.254) (layer F.Cu) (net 8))
 (segment (start 123.571 100.584) (end 124.841 101.854) (width 0.254) (layer F.Cu) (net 8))
 (segment (start 127 103.378) (end 127.127 103.505) (width 0.254) (layer F.Cu) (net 8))
 (segment (start 144.096 100.02) (end 143.042 100.02) (width 0.254) (layer F.Cu) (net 8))
 (segment (start 143.042 100.02) (end 139.557 103.505) (width 0.254) (layer F.Cu) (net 8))
 (segment (start 139.557 103.505) (end 127.127 103.505) (width 0.254) (layer F.Cu) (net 8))
 (segment (start 139.065 96.731) (end 137.711 96.731) (width 0.254) (layer F.Cu) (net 9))
 (segment (start 137.668 98.933) (end 139.954 101.219) (width 0.254) (layer B.Cu) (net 9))
 (segment (start 137.668 96.774) (end 137.668 98.933) (width 0.254) (layer B.Cu) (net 9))
 (via (at 137.668 96.774) (size 0.762) (drill 0.3302) (layers F.Cu B.Cu) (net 9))
 (segment (start 137.711 96.731) (end 137.668 96.774) (width 0.254) (layer F.Cu) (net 9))
 (segment (start 134.923 99.624) (end 138.359 99.624) (width 0.254) (layer F.Cu) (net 9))
 (segment (start 138.359 99.624) (end 139.954 101.219) (width 0.254) (layer F.Cu) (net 9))
 (segment (start 139.954 101.219) (end 140.589 101.219) (width 0.254) (layer F.Cu) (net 9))
 (segment (start 140.589 101.219) (end 142.438 99.37) (width 0.254) (layer F.Cu) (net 9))
 (segment (start 142.438 99.37) (end 144.096 99.37) (width 0.254) (layer F.Cu) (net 9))
 (segment (start 142.113 96.731) (end 142.113 98.679) (width 0.254) (layer F.Cu) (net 10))
 (segment (start 142.113 98.679) (end 142.072 98.72) (width 0.254) (layer F.Cu) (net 10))
 (segment (start 134.923 98.974) (end 139.868 98.974) (width 0.254) (layer F.Cu) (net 10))
 (segment (start 139.868 98.974) (end 139.954 99.06) (width 0.254) (layer F.Cu) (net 10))
 (segment (start 139.954 99.06) (end 141.732 99.06) (width 0.254) (layer F.Cu) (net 10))
 (segment (start 141.732 99.06) (end 142.072 98.72) (width 0.254) (layer F.Cu) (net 10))
 (segment (start 142.072 98.72) (end 144.096 98.72) (width 0.254) (layer F.Cu) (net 10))
 (segment (start 130.386 93.914) (end 130.386 94.826) (width 0.381) (layer F.Cu) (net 11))
 (segment (start 130.386 94.826) (end 131.572 96.012) (width 0.381) (layer F.Cu) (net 11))
 (segment (start 145.9484 96.9518) (end 145.9484 95.0468) (width 0.4572) (layer F.Cu) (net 12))
 (segment (start 145.9484 97.6376) (end 145.9484 96.9518) (width 0.381) (layer F.Cu) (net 12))
 (segment (start 145.9484 98.2726) (end 145.9484 97.6376) (width 0.3048) (layer F.Cu) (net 12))
 (segment (start 145.9484 98.8764) (end 145.9484 98.2726) (width 0.254) (layer F.Cu) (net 12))
 (segment (start 147.496 99.37) (end 146.442 99.37) (width 0.254) (layer F.Cu) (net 12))
 (segment (start 146.442 99.37) (end 145.9484 98.8764) (width 0.254) (layer F.Cu) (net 12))
 (segment (start 147.496 99.37) (end 147.4908 99.3648) (width 0.254) (layer F.Cu) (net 12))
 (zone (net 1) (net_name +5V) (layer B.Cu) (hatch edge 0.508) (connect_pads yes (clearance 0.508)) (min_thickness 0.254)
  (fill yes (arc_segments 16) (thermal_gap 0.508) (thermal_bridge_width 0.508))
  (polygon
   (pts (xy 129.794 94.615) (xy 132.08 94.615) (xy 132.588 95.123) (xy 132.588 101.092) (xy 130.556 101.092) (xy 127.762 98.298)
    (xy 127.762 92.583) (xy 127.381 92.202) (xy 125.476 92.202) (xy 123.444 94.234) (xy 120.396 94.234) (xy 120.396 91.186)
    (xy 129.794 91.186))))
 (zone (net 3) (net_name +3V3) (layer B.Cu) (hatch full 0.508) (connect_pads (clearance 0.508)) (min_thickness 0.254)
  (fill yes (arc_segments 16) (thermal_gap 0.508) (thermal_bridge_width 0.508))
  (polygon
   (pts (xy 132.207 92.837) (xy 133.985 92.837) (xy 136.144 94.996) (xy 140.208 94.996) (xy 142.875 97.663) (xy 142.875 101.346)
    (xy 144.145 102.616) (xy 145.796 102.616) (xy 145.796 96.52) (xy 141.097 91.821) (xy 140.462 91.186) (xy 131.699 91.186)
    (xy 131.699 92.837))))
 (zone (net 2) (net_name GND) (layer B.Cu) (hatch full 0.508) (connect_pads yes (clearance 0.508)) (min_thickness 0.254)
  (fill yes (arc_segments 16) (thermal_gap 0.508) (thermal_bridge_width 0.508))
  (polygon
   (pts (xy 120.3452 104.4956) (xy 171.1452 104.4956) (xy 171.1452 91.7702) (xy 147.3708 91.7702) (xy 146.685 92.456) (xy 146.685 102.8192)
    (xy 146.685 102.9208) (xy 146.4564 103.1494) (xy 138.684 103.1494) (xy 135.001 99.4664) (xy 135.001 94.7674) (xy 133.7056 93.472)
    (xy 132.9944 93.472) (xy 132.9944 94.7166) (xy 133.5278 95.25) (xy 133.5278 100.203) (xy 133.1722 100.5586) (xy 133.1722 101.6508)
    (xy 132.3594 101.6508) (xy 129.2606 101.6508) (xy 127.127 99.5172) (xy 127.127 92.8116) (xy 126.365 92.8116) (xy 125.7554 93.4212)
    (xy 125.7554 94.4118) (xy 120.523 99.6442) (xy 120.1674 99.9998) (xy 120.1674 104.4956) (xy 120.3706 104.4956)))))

